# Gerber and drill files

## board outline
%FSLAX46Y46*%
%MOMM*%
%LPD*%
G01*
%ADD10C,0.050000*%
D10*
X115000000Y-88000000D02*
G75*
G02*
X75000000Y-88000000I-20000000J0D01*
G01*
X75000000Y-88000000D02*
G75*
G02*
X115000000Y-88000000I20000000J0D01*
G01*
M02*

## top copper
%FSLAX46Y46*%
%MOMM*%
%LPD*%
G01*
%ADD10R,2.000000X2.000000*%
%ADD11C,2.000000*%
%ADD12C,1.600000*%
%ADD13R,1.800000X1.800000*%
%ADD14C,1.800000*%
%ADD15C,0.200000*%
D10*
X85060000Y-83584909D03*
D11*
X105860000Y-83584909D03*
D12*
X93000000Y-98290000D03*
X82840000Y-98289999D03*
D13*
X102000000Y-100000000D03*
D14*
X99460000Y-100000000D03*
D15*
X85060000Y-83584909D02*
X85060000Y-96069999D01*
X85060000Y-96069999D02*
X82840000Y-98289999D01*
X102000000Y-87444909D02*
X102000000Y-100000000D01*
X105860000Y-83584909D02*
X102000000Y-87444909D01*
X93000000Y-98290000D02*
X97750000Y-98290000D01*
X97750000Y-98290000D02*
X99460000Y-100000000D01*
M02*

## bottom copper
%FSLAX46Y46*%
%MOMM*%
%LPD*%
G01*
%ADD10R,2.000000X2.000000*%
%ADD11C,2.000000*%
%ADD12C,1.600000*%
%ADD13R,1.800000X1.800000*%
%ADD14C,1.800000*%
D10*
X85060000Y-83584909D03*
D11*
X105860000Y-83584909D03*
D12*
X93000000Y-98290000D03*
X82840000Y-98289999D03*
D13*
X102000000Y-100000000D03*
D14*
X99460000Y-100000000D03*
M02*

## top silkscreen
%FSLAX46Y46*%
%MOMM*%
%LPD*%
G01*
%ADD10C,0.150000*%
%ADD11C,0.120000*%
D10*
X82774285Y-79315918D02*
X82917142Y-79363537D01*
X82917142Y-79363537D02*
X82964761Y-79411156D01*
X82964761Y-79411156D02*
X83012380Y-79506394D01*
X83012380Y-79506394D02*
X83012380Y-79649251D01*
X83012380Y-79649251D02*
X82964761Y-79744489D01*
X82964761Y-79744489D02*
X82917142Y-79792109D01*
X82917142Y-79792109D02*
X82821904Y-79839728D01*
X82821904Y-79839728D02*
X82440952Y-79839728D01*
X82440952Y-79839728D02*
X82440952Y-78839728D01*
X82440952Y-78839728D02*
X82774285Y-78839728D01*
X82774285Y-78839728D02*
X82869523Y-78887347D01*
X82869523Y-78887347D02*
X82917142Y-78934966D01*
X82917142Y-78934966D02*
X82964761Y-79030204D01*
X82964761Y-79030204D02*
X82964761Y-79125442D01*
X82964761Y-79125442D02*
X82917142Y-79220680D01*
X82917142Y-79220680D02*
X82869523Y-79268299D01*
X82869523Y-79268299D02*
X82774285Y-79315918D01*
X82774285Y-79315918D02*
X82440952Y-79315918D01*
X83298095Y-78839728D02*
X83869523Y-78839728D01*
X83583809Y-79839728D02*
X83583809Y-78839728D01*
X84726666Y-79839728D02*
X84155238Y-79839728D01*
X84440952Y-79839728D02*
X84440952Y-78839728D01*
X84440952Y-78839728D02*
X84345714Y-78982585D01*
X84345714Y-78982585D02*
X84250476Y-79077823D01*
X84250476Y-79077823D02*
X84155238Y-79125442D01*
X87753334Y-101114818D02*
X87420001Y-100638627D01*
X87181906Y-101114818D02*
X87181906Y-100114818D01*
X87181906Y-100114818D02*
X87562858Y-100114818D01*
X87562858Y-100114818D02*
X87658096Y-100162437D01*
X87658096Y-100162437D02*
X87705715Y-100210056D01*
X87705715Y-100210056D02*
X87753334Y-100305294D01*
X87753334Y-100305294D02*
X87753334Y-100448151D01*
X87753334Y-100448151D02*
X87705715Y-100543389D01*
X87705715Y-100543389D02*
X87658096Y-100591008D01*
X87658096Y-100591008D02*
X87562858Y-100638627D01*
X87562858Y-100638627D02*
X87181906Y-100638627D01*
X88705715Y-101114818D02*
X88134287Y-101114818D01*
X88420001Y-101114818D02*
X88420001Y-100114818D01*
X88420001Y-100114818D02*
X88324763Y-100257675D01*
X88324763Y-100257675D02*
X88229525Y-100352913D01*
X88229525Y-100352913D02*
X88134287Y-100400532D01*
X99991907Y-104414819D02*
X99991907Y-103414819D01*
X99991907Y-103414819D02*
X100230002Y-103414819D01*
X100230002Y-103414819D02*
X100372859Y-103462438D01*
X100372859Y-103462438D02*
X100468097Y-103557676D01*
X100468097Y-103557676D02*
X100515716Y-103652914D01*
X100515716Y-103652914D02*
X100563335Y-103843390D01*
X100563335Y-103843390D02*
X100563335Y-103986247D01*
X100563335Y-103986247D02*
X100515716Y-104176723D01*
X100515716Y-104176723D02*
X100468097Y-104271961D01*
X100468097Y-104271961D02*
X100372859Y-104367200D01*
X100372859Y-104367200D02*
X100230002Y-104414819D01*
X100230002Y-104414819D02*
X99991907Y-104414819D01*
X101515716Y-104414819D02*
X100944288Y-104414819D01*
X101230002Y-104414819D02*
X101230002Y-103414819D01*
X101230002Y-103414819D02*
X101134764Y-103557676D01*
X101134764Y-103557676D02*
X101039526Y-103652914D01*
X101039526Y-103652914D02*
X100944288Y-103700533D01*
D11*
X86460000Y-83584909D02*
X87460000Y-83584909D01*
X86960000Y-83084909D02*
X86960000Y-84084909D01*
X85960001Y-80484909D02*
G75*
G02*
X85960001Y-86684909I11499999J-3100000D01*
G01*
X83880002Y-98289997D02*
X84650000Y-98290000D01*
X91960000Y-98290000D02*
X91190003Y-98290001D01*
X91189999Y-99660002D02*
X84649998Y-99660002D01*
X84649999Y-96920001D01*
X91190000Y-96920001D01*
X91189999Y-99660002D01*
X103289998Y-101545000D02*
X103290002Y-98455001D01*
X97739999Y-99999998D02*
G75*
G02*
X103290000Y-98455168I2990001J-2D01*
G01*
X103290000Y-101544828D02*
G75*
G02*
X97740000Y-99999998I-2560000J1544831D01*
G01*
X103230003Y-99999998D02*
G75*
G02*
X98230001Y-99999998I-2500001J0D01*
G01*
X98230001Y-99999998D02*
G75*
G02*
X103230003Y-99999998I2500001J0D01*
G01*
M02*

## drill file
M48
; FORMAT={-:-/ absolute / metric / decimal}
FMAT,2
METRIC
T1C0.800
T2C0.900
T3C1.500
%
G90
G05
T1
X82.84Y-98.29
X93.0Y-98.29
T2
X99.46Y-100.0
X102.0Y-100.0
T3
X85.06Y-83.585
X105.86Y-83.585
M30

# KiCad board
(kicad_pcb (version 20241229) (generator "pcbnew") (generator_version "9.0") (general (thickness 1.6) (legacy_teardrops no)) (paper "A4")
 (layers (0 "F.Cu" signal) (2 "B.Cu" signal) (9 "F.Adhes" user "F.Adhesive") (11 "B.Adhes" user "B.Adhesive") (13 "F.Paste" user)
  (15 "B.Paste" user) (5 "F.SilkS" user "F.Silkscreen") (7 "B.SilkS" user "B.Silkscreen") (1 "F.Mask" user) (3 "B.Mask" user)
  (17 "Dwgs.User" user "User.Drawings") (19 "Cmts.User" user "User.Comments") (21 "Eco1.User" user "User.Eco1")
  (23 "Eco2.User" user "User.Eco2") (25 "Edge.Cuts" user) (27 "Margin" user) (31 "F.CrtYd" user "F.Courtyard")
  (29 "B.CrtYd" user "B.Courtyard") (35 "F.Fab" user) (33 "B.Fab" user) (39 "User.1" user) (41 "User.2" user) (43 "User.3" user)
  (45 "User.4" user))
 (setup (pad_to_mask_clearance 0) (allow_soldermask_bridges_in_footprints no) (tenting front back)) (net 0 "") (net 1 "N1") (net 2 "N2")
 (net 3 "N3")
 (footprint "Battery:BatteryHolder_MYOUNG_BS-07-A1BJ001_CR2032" (layer "F.Cu") (at 85.06 83.584909)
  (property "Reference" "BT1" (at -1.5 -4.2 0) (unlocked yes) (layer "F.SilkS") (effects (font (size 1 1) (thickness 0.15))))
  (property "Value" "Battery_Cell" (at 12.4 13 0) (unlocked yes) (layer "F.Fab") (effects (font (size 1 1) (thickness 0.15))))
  (fp_line (start 1.4 0) (end 2.4 0) (stroke (width 0.12) (type default)) (layer "F.SilkS"))
  (fp_line (start 1.9 -0.5) (end 1.9 0.5) (stroke (width 0.12) (type default)) (layer "F.SilkS"))
  (fp_arc (start 0.900001 -3.1) (mid 24.310499 0) (end 0.900001 3.1) (stroke (width 0.12) (type default)) (layer "F.SilkS"))
  (pad "1" thru_hole rect (at 0 0 180) (size 2 2) (drill 1.5) (layers "*.Cu" "*.Mask") (remove_unused_layers no) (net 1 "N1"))
  (pad "2" thru_hole circle (at 20.8 0 180) (size 2 2) (drill 1.5) (layers "*.Cu" "*.Mask") (remove_unused_layers no) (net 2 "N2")))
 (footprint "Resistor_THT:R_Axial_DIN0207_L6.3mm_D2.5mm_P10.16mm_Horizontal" (layer "F.Cu") (at 93 98.29 180)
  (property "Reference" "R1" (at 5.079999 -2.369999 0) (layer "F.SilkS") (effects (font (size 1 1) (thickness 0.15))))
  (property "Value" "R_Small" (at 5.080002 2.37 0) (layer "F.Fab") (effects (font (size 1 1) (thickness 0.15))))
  (fp_line (start 9.119998 0.000003) (end 8.35 0) (stroke (width 0.12) (type solid)) (layer "F.SilkS"))
  (fp_line (start 1.04 0) (end 1.809997 -0.000001) (stroke (width 0.12) (type solid)) (layer "F.SilkS"))
  (fp_poly
   (pts (xy 1.810001 -1.370002) (xy 8.350002 -1.370002) (xy 8.350001 1.369999) (xy 1.81 1.369999)) (stroke (width 0.12) (type solid))
   (fill no) (layer "F.SilkS"))
  (pad "1" thru_hole circle (at 0 0 180) (size 1.6 1.6) (drill 0.8) (layers "*.Cu" "*.Mask") (remove_unused_layers no) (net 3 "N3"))
  (pad "2" thru_hole circle (at 10.16 0.000001 180) (size 1.6 1.6) (drill 0.8) (layers "*.Cu" "*.Mask") (remove_unused_layers no)
   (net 1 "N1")))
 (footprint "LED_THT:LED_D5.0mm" (layer "F.Cu") (at 102 100 180)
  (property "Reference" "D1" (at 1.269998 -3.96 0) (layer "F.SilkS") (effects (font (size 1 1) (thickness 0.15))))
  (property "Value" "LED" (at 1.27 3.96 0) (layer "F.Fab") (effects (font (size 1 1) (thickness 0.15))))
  (fp_line (start -1.289998 -1.545) (end -1.290002 1.544999) (stroke (width 0.12) (type solid)) (layer "F.SilkS"))
  (fp_arc (start 4.260001 0.000002) (mid 2.071779 2.880496) (end -1.29 1.544832) (stroke (width 0.12) (type solid)) (layer "F.SilkS"))
  (fp_arc (start -1.29 -1.544828) (mid 2.071779 -2.880493) (end 4.260001 0.000002) (stroke (width 0.12) (type solid)) (layer "F.SilkS"))
  (fp_circle (center 1.269998 0.000002) (end 3.769999 0.000002) (stroke (width 0.12) (type solid)) (fill no) (layer "F.SilkS"))
  (pad "1" thru_hole rect (at 0 0 180) (size 1.8 1.8) (drill 0.9) (layers "*.Cu" "*.Mask") (remove_unused_layers no) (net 2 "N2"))
  (pad "2" thru_hole circle (at 2.54 0 180) (size 1.8 1.8) (drill 0.9) (layers "*.Cu" "*.Mask") (remove_unused_layers no) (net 3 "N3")))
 (gr_circle (center 95 88) (end 115 88) (stroke (width 0.05) (type default)) (fill no) (layer "Edge.Cuts"))
 (segment (start 85.06 83.584909) (end 85.06 96.069999) (width 0.2) (layer "F.Cu") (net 1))
 (segment (start 85.06 96.069999) (end 82.84 98.289999) (width 0.2) (layer "F.Cu") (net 1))
 (segment (start 102 87.444909) (end 102 100) (width 0.2) (layer "F.Cu") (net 2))
 (segment (start 105.86 83.584909) (end 102 87.444909) (width 0.2) (layer "F.Cu") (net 2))
 (segment (start 93 98.29) (end 97.75 98.29) (width 0.2) (layer "F.Cu") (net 3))
 (segment (start 97.75 98.29) (end 99.46 100) (width 0.2) (layer "F.Cu") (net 3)))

